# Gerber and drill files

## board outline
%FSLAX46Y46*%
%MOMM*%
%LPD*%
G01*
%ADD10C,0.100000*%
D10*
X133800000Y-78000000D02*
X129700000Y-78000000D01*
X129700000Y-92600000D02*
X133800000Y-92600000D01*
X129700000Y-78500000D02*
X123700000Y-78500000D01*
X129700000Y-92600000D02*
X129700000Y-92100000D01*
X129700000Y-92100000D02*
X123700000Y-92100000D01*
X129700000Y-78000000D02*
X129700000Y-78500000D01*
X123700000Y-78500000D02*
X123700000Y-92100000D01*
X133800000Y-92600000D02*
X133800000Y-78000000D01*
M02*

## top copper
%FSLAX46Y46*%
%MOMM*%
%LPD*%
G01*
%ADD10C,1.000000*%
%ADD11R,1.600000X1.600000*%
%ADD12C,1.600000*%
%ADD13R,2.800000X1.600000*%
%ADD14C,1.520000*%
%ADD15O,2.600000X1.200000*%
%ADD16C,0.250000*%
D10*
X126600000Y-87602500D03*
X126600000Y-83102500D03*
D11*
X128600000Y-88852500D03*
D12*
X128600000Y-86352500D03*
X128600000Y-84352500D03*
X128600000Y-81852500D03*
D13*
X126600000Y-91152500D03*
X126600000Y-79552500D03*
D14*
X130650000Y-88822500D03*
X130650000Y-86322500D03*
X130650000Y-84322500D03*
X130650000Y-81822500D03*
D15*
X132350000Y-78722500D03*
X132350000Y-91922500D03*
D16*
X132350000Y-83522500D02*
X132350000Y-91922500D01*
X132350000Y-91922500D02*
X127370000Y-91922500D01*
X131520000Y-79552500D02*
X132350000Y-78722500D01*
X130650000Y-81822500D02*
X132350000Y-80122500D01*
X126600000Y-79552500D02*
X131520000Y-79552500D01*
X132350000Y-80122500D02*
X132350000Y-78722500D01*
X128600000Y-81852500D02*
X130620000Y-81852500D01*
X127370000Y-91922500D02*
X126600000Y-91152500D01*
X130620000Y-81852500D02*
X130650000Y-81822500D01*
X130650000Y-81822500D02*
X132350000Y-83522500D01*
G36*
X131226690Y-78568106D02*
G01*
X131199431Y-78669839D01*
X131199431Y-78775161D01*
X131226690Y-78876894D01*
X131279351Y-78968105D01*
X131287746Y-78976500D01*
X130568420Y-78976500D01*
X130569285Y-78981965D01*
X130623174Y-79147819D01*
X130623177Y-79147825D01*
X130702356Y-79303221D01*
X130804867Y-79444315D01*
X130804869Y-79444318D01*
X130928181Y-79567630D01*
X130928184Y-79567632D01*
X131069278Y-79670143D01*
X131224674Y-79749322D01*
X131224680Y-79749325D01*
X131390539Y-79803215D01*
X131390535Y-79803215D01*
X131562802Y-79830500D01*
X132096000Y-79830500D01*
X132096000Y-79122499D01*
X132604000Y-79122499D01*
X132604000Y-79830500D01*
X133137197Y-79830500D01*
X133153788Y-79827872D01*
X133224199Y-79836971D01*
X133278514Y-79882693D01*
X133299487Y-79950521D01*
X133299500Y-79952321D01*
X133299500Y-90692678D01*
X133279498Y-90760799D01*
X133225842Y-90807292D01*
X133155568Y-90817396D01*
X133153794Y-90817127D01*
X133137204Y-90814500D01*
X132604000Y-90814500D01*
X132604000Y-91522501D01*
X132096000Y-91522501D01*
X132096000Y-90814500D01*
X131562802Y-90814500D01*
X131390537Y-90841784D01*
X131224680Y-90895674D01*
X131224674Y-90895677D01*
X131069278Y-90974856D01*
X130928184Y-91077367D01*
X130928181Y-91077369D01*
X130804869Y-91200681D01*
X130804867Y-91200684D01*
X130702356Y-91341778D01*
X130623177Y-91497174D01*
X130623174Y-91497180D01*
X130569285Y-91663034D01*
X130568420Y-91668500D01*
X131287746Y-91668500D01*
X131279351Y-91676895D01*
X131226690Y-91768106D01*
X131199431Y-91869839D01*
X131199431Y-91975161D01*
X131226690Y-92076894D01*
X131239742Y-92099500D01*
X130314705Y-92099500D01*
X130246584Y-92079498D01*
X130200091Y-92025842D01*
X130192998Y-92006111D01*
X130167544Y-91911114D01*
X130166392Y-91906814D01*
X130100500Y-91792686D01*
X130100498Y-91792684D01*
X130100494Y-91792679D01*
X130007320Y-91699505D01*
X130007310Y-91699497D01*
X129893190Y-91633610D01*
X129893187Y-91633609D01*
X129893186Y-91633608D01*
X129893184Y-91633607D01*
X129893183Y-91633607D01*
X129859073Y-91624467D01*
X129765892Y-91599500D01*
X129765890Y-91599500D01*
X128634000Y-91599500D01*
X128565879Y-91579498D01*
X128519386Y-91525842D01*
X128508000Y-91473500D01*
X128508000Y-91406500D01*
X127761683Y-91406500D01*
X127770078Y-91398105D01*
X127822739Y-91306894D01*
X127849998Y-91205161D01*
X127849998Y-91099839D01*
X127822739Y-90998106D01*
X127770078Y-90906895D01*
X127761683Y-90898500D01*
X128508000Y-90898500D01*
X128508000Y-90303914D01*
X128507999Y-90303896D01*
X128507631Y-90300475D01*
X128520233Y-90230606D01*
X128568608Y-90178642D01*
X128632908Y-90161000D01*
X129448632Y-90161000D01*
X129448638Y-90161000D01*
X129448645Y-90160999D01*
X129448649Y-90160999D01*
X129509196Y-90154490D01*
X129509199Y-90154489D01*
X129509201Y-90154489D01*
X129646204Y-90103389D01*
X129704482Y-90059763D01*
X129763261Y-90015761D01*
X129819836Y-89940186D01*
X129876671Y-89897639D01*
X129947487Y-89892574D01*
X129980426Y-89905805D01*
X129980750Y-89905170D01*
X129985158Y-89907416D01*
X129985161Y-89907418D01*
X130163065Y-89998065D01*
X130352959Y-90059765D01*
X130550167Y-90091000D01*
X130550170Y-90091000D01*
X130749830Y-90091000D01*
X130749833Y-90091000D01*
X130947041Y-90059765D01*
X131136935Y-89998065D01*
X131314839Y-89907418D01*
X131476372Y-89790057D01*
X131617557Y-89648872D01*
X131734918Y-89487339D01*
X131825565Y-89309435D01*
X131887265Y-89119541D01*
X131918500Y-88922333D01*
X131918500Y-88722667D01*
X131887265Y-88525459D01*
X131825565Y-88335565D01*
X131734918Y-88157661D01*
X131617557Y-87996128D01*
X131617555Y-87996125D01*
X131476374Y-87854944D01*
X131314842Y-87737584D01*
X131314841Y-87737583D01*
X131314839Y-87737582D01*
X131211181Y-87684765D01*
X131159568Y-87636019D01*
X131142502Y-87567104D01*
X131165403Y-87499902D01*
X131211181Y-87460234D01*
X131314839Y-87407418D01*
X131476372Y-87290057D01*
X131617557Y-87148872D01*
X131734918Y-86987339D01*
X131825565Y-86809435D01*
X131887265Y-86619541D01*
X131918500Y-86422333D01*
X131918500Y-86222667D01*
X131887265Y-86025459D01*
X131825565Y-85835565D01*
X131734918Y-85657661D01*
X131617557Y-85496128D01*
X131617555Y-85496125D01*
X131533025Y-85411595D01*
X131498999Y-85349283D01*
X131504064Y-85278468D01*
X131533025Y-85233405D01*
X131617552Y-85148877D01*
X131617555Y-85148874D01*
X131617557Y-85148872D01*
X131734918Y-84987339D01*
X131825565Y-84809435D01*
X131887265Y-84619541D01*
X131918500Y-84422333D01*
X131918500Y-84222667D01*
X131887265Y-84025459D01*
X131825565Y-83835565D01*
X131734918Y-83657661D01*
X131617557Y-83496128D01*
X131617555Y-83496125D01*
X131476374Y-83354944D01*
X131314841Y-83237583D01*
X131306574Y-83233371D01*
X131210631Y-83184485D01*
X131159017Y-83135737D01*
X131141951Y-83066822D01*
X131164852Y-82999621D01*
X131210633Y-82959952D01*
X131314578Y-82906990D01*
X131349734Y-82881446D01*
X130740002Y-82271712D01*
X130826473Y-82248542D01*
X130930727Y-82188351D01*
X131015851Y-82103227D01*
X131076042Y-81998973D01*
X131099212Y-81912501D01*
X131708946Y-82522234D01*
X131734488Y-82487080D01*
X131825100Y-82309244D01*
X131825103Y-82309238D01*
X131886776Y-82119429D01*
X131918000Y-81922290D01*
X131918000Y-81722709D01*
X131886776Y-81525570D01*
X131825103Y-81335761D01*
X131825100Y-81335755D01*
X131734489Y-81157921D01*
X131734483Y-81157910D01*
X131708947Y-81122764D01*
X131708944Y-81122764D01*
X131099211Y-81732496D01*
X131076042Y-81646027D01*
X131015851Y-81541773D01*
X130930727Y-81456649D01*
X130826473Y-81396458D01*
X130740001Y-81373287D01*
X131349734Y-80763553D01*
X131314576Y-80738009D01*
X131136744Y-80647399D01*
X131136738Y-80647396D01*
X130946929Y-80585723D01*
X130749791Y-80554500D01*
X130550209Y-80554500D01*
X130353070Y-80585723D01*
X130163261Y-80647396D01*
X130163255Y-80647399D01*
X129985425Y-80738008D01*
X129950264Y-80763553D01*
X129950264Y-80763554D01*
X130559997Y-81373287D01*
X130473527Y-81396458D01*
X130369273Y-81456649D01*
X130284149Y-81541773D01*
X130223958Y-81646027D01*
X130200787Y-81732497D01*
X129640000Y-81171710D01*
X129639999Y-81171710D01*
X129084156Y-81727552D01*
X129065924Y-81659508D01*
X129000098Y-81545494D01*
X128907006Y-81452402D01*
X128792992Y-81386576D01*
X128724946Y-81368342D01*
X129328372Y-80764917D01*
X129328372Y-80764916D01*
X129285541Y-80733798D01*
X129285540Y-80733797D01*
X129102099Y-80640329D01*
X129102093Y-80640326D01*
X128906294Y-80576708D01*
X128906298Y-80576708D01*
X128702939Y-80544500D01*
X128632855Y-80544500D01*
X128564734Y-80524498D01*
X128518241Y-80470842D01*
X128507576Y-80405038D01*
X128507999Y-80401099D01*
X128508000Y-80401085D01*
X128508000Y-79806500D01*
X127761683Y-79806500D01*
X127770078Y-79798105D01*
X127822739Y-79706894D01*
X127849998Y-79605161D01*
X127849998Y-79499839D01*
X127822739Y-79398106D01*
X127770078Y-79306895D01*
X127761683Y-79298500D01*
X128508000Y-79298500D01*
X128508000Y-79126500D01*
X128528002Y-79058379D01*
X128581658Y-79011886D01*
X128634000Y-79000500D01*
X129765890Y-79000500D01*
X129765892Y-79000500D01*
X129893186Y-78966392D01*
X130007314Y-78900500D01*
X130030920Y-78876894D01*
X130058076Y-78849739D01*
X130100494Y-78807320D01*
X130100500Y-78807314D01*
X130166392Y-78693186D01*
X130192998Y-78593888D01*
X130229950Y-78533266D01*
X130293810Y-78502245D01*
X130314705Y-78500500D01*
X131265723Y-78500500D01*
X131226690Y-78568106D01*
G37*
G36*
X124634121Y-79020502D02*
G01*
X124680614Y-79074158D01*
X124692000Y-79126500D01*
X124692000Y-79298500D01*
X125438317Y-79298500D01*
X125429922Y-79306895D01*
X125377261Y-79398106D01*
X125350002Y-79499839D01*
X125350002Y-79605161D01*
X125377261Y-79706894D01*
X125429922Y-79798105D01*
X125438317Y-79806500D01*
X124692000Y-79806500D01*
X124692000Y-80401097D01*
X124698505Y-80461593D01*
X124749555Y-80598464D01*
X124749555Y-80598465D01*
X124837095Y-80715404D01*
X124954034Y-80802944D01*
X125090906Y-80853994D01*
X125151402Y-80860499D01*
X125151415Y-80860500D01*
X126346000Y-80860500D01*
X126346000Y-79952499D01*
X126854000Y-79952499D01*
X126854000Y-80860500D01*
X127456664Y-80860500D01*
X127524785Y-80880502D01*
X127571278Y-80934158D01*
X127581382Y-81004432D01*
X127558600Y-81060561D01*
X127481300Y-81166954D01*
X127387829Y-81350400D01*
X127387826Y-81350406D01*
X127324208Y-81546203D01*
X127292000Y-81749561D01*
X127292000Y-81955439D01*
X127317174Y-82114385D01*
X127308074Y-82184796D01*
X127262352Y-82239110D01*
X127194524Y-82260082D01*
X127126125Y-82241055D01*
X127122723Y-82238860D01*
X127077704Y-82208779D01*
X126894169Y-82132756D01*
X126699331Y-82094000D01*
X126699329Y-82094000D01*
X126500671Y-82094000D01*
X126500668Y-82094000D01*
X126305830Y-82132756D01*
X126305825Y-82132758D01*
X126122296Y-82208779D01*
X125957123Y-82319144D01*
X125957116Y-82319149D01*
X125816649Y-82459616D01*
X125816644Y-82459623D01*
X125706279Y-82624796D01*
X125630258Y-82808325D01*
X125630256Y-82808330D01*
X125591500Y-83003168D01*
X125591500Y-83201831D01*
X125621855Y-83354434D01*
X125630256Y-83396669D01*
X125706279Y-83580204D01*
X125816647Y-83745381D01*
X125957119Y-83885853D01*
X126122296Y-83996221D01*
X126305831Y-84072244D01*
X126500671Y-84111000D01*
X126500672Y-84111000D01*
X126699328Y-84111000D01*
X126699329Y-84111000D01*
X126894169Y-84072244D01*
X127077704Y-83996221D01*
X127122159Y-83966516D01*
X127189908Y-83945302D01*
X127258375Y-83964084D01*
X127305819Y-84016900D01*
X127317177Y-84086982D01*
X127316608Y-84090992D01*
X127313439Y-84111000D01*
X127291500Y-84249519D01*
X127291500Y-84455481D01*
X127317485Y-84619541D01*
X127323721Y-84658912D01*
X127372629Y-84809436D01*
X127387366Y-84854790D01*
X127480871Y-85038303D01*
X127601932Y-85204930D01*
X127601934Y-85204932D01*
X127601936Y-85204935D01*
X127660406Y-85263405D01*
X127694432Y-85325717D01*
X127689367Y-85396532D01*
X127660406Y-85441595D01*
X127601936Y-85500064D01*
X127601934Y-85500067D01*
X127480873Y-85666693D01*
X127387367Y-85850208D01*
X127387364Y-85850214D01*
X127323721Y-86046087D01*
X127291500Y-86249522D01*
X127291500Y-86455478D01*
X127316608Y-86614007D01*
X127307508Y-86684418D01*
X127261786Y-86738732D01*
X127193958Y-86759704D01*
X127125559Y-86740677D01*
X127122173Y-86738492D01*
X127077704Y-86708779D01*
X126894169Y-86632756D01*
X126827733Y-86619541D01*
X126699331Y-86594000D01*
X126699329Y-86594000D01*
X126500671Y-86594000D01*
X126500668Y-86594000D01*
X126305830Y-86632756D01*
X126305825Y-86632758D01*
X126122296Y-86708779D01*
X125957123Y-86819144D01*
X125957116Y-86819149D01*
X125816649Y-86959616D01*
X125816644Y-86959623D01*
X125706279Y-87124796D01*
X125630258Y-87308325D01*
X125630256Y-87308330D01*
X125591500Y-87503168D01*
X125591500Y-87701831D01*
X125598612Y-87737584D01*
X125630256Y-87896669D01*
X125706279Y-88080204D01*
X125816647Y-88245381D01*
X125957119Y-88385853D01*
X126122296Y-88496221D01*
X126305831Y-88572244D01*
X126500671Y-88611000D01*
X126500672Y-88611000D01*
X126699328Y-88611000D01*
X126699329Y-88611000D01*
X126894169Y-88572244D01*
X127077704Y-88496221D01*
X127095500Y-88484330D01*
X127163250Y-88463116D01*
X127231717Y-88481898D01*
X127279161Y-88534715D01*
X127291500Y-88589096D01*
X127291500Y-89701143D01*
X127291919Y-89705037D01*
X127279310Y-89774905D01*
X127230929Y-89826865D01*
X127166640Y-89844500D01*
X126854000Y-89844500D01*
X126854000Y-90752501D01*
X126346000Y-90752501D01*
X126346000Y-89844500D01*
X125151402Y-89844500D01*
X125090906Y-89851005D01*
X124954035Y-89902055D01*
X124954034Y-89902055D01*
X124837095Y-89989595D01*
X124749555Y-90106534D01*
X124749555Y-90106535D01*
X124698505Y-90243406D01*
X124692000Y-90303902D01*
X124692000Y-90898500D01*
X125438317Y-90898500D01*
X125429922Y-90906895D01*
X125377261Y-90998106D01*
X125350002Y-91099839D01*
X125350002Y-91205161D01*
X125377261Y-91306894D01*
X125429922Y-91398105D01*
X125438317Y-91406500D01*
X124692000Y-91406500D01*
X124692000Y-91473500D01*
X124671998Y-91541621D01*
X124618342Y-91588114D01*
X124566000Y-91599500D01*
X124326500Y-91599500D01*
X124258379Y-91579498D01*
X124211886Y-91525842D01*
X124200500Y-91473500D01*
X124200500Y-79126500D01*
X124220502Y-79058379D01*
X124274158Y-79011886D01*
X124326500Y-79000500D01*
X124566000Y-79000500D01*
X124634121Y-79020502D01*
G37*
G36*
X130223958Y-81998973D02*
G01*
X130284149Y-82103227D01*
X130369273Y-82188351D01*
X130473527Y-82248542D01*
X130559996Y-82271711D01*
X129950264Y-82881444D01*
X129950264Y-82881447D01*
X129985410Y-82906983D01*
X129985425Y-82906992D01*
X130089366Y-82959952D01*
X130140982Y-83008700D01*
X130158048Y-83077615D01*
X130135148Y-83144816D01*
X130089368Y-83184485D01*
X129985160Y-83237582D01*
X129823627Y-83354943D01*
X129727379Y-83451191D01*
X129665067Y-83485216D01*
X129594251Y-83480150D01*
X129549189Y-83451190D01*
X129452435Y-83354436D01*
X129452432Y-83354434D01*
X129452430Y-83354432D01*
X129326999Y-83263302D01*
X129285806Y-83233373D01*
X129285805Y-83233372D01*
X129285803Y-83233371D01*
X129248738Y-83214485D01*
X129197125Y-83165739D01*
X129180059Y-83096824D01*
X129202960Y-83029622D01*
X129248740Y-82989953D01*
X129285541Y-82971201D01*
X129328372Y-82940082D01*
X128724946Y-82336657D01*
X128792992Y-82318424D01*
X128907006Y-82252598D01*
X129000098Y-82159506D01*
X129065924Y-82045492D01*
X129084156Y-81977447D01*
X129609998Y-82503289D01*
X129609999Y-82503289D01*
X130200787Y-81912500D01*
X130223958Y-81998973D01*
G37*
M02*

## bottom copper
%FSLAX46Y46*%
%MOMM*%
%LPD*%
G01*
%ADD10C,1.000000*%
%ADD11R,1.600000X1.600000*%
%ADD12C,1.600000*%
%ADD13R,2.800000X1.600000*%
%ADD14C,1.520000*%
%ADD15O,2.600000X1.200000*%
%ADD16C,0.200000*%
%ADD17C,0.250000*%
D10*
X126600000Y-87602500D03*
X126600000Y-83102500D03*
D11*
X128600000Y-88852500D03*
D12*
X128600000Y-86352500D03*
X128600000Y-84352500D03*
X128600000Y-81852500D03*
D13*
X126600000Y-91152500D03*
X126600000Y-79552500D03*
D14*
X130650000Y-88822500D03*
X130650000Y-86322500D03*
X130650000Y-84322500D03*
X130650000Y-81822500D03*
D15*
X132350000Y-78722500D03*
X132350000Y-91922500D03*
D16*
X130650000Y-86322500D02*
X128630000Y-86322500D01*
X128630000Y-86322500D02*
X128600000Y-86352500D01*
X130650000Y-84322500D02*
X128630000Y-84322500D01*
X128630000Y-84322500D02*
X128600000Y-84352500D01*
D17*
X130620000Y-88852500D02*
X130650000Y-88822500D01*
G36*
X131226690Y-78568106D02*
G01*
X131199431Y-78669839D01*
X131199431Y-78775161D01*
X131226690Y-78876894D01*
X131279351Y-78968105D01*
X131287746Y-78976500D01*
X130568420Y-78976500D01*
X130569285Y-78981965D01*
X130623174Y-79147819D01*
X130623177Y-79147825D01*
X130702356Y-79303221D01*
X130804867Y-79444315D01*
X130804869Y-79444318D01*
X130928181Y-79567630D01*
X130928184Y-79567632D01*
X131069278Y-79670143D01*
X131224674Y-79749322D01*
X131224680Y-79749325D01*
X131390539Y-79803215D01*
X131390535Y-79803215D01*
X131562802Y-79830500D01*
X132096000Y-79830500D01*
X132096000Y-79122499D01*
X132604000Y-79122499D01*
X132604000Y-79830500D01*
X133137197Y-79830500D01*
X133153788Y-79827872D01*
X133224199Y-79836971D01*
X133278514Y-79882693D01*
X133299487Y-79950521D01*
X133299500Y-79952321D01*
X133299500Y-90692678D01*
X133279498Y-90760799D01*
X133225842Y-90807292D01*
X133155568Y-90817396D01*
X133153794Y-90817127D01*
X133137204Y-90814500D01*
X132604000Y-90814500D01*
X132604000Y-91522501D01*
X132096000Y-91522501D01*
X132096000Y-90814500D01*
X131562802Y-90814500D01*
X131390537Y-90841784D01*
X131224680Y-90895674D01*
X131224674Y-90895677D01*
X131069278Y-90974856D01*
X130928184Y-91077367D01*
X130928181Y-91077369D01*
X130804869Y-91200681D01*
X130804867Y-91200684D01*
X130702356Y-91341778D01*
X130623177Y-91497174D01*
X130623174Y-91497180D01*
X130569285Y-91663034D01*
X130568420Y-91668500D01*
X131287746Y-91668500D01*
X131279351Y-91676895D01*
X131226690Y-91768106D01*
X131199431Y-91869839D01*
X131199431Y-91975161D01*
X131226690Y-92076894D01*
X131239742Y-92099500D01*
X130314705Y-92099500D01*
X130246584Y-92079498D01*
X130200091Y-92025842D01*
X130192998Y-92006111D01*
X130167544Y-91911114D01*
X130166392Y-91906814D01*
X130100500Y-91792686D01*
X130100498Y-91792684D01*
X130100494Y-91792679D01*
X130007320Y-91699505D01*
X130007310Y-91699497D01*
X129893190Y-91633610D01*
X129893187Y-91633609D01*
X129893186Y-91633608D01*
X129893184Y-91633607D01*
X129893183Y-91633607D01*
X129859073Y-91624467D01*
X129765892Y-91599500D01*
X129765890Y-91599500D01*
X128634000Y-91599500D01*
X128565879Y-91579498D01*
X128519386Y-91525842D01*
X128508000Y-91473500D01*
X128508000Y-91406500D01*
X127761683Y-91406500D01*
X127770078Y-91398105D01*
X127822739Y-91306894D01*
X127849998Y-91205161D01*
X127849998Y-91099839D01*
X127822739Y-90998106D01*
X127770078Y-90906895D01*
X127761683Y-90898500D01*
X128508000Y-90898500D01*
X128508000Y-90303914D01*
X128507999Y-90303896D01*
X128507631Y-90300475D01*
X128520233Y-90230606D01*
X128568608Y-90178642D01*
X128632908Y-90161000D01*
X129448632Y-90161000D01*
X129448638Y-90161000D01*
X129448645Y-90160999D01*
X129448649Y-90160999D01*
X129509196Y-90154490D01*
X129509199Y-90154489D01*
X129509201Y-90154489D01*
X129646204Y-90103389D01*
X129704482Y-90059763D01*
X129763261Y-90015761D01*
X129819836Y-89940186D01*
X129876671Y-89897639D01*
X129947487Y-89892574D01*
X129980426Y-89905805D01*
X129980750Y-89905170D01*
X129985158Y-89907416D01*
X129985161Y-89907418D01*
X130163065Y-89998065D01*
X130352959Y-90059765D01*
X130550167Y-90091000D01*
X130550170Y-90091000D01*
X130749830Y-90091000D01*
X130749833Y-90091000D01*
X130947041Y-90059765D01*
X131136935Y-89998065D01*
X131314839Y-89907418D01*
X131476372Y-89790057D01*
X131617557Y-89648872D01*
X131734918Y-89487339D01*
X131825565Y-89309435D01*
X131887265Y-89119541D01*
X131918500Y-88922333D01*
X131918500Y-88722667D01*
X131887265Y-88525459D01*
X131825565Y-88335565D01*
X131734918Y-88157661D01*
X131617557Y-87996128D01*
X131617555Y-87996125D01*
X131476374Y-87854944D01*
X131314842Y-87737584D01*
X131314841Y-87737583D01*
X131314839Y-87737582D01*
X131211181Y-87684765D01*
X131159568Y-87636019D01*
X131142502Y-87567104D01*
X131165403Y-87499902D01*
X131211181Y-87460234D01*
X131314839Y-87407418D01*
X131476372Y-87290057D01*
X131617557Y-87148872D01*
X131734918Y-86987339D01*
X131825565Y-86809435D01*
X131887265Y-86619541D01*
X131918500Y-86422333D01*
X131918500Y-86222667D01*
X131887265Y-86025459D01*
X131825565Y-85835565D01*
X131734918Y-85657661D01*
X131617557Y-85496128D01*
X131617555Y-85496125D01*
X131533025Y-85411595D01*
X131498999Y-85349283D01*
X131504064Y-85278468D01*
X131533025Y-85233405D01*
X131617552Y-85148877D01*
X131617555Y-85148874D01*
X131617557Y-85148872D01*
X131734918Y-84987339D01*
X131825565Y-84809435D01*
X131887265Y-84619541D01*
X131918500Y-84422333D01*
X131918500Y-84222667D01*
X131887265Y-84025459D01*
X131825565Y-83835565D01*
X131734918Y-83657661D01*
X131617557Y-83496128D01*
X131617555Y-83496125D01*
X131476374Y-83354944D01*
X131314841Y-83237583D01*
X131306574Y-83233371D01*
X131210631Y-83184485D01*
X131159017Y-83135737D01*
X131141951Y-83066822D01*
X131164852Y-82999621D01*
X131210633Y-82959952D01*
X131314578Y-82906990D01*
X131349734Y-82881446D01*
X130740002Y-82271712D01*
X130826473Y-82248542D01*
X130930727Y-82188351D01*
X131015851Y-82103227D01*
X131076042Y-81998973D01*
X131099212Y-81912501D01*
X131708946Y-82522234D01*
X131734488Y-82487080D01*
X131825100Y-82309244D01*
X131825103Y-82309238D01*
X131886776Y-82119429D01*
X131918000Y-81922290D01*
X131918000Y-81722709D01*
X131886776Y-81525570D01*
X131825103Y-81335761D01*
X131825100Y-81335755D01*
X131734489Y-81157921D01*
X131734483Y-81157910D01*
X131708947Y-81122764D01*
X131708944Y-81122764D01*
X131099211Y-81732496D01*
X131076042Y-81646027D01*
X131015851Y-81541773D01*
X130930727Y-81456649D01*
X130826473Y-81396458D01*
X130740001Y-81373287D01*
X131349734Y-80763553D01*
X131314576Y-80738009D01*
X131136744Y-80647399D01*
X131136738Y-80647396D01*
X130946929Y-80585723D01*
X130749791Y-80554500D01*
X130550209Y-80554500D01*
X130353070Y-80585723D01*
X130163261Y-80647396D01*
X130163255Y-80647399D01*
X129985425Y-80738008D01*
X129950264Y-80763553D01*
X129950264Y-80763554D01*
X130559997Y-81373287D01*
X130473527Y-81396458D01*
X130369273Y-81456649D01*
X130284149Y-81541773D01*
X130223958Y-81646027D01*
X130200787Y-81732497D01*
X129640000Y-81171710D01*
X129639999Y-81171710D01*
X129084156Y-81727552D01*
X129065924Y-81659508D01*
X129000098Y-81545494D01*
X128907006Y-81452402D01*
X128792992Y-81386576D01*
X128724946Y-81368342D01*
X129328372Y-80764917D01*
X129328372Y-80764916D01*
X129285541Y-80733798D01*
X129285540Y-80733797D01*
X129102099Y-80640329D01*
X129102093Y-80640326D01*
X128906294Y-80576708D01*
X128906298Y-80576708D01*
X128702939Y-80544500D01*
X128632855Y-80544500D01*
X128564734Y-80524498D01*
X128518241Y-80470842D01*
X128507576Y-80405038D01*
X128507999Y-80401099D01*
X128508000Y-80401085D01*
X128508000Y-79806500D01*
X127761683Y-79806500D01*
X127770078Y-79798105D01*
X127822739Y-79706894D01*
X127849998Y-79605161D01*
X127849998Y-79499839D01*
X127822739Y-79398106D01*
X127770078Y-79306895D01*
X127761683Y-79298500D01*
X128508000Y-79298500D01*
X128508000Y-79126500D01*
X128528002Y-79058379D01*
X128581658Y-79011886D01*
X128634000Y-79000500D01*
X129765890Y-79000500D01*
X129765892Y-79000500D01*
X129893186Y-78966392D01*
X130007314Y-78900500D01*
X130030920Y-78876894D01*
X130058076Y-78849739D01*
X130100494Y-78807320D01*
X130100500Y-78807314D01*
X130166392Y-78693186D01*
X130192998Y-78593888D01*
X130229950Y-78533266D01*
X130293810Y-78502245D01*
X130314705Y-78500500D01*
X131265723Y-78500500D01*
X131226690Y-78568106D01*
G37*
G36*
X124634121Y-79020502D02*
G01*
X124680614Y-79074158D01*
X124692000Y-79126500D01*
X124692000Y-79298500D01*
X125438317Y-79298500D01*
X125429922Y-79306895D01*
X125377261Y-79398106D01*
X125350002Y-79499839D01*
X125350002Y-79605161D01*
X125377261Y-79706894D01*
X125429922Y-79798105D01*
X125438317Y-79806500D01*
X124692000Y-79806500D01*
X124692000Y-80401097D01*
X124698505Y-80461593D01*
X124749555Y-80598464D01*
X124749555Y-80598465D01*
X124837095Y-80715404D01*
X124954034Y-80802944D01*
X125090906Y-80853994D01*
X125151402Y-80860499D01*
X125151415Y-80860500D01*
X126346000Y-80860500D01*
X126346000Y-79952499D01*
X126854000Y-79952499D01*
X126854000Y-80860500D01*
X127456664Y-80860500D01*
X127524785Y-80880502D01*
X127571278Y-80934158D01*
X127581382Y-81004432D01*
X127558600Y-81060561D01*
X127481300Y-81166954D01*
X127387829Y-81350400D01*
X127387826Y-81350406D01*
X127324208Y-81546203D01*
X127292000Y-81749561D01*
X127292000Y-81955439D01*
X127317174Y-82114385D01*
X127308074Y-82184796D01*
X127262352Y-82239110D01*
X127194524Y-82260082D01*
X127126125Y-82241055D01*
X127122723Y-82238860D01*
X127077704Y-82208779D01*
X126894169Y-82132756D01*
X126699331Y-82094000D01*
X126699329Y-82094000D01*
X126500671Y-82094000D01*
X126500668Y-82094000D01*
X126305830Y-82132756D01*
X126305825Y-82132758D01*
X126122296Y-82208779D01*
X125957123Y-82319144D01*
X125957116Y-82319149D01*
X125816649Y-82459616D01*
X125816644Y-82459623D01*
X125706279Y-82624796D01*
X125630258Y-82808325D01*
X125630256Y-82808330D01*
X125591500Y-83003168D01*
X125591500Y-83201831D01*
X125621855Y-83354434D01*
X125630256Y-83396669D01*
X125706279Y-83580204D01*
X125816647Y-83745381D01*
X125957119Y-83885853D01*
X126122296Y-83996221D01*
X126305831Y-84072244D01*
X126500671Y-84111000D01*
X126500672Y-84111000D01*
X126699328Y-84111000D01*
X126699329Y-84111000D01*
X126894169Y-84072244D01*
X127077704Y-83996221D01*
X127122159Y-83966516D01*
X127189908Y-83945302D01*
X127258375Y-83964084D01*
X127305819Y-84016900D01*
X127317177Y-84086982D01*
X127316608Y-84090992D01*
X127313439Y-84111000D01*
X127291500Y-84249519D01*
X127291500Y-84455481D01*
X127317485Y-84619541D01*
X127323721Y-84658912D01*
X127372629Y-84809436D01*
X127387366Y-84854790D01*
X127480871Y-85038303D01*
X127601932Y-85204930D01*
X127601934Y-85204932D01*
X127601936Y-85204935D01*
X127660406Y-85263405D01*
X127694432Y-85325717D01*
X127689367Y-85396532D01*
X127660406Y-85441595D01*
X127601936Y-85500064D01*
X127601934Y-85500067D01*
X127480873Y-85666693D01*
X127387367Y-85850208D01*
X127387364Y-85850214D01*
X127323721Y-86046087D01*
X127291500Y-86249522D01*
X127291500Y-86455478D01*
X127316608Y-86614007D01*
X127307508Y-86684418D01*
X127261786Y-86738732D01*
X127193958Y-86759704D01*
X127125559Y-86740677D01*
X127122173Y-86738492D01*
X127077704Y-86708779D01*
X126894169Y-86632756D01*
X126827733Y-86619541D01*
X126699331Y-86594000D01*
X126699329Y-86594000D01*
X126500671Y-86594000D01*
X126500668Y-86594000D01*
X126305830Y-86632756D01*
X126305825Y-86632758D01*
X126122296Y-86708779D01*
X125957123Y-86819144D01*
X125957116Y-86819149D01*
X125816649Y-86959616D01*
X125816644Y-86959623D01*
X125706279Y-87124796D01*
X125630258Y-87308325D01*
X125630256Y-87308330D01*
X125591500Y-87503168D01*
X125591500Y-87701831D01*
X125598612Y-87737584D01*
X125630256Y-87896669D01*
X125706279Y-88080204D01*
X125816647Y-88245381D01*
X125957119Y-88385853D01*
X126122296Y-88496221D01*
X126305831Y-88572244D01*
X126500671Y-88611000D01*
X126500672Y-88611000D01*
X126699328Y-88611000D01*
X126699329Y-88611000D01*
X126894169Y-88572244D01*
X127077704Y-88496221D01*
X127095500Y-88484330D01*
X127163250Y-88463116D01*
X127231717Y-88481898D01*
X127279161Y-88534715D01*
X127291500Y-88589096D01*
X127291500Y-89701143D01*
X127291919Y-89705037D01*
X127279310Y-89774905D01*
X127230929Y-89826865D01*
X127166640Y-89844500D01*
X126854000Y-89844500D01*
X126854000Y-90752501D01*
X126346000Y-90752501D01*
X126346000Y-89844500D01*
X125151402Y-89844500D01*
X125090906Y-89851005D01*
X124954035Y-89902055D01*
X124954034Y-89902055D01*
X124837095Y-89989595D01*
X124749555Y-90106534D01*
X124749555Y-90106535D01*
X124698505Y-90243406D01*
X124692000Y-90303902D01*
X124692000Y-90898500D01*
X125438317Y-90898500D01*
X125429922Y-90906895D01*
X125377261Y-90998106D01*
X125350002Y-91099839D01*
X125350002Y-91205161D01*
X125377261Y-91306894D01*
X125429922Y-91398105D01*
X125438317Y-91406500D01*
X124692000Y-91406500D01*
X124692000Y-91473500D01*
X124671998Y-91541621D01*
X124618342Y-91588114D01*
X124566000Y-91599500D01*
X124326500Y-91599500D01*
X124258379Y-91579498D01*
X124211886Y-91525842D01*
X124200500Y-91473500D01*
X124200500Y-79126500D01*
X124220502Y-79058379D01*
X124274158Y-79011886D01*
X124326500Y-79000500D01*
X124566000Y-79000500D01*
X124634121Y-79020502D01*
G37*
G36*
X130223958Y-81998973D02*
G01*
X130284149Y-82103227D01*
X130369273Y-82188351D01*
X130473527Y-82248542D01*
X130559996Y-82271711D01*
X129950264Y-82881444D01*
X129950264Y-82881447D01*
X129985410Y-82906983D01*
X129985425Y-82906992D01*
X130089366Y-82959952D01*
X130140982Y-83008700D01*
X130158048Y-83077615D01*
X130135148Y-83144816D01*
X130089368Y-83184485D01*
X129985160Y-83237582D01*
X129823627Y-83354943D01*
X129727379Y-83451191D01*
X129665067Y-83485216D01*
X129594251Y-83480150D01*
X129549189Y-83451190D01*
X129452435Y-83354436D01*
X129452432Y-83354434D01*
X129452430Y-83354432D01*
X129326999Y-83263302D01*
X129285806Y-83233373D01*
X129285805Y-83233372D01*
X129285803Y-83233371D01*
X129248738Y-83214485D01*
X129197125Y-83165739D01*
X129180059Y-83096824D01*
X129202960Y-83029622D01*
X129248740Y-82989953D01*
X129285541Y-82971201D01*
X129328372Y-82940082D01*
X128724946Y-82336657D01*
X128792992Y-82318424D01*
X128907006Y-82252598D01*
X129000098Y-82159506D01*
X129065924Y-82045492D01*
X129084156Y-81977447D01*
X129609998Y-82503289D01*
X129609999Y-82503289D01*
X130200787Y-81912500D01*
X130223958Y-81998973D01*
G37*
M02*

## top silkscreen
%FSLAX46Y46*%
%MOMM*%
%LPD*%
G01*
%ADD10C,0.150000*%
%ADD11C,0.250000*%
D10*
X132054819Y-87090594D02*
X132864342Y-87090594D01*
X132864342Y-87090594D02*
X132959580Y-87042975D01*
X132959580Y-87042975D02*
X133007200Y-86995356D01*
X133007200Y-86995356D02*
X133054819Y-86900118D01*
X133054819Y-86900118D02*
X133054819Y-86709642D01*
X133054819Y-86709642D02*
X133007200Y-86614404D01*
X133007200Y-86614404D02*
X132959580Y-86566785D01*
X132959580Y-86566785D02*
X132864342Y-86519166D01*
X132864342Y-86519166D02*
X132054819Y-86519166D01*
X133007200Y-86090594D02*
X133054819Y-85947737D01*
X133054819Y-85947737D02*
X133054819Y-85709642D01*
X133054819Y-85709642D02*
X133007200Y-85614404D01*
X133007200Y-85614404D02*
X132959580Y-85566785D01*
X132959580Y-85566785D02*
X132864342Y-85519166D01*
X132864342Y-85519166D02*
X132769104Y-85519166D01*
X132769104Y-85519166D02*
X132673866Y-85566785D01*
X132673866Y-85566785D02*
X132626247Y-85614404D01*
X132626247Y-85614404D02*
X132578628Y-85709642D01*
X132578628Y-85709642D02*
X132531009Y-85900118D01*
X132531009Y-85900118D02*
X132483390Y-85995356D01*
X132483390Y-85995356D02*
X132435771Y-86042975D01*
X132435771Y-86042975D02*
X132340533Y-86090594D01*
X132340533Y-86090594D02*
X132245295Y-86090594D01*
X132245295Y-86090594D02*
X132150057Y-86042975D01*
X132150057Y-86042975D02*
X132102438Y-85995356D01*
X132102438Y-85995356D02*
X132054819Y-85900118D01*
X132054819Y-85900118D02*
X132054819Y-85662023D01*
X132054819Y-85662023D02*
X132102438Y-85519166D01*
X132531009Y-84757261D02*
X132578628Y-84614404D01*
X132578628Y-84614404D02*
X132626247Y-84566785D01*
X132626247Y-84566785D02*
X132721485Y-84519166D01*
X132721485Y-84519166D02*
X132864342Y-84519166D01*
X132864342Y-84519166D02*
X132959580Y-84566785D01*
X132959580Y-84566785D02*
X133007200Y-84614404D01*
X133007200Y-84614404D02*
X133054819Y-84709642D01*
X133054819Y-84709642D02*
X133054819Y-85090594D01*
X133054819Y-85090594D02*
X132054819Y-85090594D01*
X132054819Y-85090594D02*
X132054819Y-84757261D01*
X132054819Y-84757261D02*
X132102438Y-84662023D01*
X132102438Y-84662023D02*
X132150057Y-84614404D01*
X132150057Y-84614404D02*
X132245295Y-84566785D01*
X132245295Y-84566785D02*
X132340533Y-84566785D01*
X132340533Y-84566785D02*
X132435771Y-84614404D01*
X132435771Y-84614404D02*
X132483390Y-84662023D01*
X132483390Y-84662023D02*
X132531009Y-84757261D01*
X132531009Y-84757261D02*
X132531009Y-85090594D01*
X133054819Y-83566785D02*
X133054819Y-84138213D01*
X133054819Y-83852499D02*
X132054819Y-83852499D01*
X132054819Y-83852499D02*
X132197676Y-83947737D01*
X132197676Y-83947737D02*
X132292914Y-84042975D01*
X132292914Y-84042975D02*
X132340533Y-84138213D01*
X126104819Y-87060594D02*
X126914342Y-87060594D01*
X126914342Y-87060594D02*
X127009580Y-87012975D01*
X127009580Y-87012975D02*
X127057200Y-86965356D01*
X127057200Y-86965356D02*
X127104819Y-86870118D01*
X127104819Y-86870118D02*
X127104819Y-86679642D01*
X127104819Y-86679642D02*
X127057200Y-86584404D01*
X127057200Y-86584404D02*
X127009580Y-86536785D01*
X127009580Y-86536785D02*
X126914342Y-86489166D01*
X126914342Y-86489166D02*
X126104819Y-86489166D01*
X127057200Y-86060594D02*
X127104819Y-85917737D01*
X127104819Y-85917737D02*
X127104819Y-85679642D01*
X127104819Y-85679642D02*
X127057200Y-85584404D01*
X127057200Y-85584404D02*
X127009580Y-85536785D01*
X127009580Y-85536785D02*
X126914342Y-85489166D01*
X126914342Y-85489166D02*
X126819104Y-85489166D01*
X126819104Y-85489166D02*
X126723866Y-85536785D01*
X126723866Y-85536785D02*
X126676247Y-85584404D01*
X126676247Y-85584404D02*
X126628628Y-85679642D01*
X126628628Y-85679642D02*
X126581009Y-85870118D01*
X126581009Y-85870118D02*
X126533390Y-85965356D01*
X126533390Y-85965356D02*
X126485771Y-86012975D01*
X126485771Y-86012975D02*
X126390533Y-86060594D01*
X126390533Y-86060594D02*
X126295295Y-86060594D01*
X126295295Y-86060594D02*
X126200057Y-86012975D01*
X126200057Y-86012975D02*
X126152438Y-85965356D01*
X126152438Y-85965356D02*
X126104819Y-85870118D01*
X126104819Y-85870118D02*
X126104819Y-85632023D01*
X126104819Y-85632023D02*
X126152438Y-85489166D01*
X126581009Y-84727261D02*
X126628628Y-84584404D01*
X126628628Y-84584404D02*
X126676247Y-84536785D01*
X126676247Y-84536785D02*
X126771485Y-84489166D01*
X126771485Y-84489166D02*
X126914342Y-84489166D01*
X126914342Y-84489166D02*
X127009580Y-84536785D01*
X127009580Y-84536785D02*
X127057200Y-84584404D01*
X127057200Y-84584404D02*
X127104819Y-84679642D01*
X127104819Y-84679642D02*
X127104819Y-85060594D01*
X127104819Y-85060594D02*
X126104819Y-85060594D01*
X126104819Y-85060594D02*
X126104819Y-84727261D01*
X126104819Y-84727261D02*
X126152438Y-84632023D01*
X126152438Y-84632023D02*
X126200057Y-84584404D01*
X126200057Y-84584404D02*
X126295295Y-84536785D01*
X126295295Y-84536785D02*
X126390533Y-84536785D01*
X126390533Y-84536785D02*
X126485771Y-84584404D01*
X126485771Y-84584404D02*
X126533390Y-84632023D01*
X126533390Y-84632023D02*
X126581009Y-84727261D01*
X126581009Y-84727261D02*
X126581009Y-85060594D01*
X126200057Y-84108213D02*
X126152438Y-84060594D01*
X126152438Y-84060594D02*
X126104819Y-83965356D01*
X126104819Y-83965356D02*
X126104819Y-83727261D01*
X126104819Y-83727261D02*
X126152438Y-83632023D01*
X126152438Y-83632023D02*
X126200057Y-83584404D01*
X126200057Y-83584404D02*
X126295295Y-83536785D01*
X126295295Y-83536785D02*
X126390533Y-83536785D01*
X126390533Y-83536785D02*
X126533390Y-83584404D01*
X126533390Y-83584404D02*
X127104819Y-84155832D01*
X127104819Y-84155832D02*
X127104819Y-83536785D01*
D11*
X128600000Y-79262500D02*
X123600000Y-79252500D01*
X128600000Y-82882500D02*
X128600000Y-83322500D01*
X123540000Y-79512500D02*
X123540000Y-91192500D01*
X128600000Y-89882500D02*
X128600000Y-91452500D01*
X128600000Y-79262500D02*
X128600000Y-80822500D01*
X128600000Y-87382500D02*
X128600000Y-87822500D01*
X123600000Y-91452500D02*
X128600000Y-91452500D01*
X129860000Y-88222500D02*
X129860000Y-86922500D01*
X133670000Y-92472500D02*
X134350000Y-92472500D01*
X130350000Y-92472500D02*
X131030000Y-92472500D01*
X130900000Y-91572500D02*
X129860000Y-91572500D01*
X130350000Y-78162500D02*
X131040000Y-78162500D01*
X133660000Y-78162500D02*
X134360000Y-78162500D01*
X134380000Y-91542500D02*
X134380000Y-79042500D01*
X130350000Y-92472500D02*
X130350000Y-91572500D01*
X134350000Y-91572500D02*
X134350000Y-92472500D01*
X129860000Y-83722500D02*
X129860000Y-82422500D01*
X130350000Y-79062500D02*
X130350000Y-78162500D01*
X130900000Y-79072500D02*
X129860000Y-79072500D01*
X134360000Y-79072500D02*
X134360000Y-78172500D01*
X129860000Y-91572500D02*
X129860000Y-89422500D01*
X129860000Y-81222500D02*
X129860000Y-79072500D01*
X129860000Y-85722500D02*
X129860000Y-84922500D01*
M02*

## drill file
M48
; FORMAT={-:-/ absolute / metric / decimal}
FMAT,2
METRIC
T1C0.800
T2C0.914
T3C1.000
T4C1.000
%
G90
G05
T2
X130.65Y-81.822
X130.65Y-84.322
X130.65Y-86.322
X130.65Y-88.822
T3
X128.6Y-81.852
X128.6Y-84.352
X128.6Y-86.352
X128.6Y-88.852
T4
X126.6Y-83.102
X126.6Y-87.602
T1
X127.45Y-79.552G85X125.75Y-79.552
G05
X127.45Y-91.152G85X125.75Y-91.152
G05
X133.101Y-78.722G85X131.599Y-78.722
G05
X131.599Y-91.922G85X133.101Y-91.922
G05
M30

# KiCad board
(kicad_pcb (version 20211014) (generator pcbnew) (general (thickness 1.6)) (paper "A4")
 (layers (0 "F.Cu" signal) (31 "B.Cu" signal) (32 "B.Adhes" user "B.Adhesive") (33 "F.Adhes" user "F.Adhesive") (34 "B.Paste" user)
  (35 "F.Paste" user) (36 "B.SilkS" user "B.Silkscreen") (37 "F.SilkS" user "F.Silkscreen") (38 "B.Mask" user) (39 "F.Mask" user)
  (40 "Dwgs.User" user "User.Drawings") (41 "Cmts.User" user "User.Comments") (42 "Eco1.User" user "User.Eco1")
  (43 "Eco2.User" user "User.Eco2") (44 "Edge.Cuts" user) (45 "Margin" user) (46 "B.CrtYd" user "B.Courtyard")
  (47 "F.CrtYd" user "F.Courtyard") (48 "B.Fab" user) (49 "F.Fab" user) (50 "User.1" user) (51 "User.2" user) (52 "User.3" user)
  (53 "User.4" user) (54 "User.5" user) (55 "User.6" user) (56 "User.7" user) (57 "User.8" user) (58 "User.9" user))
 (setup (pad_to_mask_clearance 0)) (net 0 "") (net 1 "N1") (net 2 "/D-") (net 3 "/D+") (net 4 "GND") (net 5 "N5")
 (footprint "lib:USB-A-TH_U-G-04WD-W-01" (layer "F.Cu") (at 127.6 85.3525 -90)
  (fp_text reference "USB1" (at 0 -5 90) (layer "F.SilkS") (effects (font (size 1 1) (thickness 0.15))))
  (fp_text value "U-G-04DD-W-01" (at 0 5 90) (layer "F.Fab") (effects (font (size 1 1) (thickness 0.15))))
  (fp_line (start -6.09 -1) (end -6.1 4) (layer "F.SilkS") (width 0.25))
  (fp_line (start -2.47 -1) (end -2.03 -1) (layer "F.SilkS") (width 0.25))
  (fp_line (start -5.84 4.06) (end 5.84 4.06) (layer "F.SilkS") (width 0.25))
  (fp_line (start 4.53 -1) (end 6.1 -1) (layer "F.SilkS") (width 0.25))
  (fp_line (start -6.09 -1) (end -4.53 -1) (layer "F.SilkS") (width 0.25))
  (fp_line (start 2.03 -1) (end 2.47 -1) (layer "F.SilkS") (width 0.25))
  (fp_line (start 6.1 4) (end 6.1 -1) (layer "F.SilkS") (width 0.25))
  (pad "" thru_hole circle (at 2.25 1 270) (size 1 1) (drill 1) (layers *.Cu *.Mask))
  (pad "" thru_hole circle (at -2.25 1 270) (size 1 1) (drill 1) (layers *.Cu *.Mask))
  (pad "1" thru_hole rect (at 3.5 -1 270) (size 1.6 1.6) (drill 0.999998) (layers *.Cu *.Paste *.Mask) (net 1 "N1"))
  (pad "2" thru_hole circle (at 1 -1 270) (size 1.6 1.6) (drill 0.999998) (layers *.Cu *.Paste *.Mask) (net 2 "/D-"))
  (pad "3" thru_hole circle (at -1 -1 270) (size 1.6 1.6) (drill 0.999998) (layers *.Cu *.Paste *.Mask) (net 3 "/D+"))
  (pad "4" thru_hole circle (at -3.5 -1 270) (size 1.6 1.6) (drill 0.999998) (layers *.Cu *.Paste *.Mask) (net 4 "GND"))
  (pad "5" thru_hole rect (at 5.8 1 270) (size 1.6 2.8) (drill oval 0.799998 2.499995) (layers *.Cu *.Paste *.Mask) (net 4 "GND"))
  (pad "6" thru_hole rect (at -5.8 1 270) (size 1.6 2.8) (drill oval 0.799998 2.499995) (layers *.Cu *.Paste *.Mask) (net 4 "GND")))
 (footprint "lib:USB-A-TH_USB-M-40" (layer "F.Cu") (at 131.5 85.3225 90)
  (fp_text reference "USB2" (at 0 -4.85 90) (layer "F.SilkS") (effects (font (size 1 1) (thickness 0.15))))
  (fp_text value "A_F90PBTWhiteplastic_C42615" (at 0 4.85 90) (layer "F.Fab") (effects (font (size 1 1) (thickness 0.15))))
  (fp_line (start -2.9 -1.64) (end -1.6 -1.64) (layer "F.SilkS") (width 0.25))
  (fp_line (start -7.15 2.17) (end -7.15 2.85) (layer "F.SilkS") (width 0.25))
  (fp_line (start -7.15 -1.15) (end -7.15 -0.47) (layer "F.SilkS") (width 0.25))
  (fp_line (start -6.25 -0.6) (end -6.25 -1.64) (layer "F.SilkS") (width 0.25))
  (fp_line (start 7.16 -1.15) (end 7.16 -0.46) (layer "F.SilkS") (width 0.25))
  (fp_line (start 7.16 2.16) (end 7.16 2.86) (layer "F.SilkS") (width 0.25))
  (fp_line (start -6.22 2.88) (end 6.28 2.88) (layer "F.SilkS") (width 0.25))
  (fp_line (start -7.15 -1.15) (end -6.25 -1.15) (layer "F.SilkS") (width 0.25))
  (fp_line (start -6.25 2.85) (end -7.15 2.85) (layer "F.SilkS") (width 0.25))
  (fp_line (start 1.6 -1.64) (end 2.9 -1.64) (layer "F.SilkS") (width 0.25))
  (fp_line (start 6.26 -1.15) (end 7.16 -1.15) (layer "F.SilkS") (width 0.25))
  (fp_line (start 6.25 -0.6) (end 6.25 -1.64) (layer "F.SilkS") (width 0.25))
  (fp_line (start 6.25 2.86) (end 7.15 2.86) (layer "F.SilkS") (width 0.25))
  (fp_line (start -6.25 -1.64) (end -4.1 -1.64) (layer "F.SilkS") (width 0.25))
  (fp_line (start 4.1 -1.64) (end 6.25 -1.64) (layer "F.SilkS") (width 0.25))
  (fp_line (start -0.4 -1.64) (end 0.4 -1.64) (layer "F.SilkS") (width 0.25))
  (pad "1" thru_hole circle (at -3.5 -0.85 90) (size 1.52 1.52) (drill 0.9144) (layers *.Cu *.Paste *.Mask) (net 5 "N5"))
  (pad "2" thru_hole circle (at -1 -0.85 90) (size 1.52 1.52) (drill 0.9144) (layers *.Cu *.Paste *.Mask) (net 2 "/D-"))
  (pad "3" thru_hole circle (at 1 -0.85 90) (size 1.52 1.52) (drill 0.9144) (layers *.Cu *.Paste *.Mask) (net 3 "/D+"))
  (pad "4" thru_hole circle (at 3.5 -0.85 90) (size 1.52 1.52) (drill 0.9144) (layers *.Cu *.Paste *.Mask) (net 4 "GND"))
  (pad "5" thru_hole oval (at 6.6 0.85 180) (size 2.6 1.2) (drill oval 2.301138 0.799998) (layers *.Cu *.Paste *.Mask) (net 4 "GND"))
  (pad "6" thru_hole oval (at -6.6 0.85) (size 2.6 1.2) (drill oval 2.301138 0.799998) (layers *.Cu *.Paste *.Mask) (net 4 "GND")))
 (gr_line (start 133.8 78) (end 129.7 78) (layer "Edge.Cuts") (width 0.1))
 (gr_line (start 129.7 92.6) (end 133.8 92.6) (layer "Edge.Cuts") (width 0.1))
 (gr_line (start 129.7 78.5) (end 123.7 78.5) (layer "Edge.Cuts") (width 0.1))
 (gr_line (start 129.7 92.6) (end 129.7 92.1) (layer "Edge.Cuts") (width 0.1))
 (gr_line (start 129.7 92.1) (end 123.7 92.1) (layer "Edge.Cuts") (width 0.1))
 (gr_line (start 129.7 78) (end 129.7 78.5) (layer "Edge.Cuts") (width 0.1))
 (gr_line (start 123.7 78.5) (end 123.7 92.1) (layer "Edge.Cuts") (width 0.1))
 (gr_line (start 133.8 92.6) (end 133.8 78) (layer "Edge.Cuts") (width 0.1))
 (segment (start 132.35 83.5225) (end 132.35 91.9225) (width 0.25) (layer "F.Cu") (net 4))
 (segment (start 132.35 91.9225) (end 127.37 91.9225) (width 0.25) (layer "F.Cu") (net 4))
 (segment (start 131.52 79.5525) (end 132.35 78.7225) (width 0.25) (layer "F.Cu") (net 4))
 (segment (start 130.65 81.8225) (end 132.35 80.1225) (width 0.25) (layer "F.Cu") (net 4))
 (segment (start 126.6 79.5525) (end 131.52 79.5525) (width 0.25) (layer "F.Cu") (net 4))
 (segment (start 132.35 80.1225) (end 132.35 78.7225) (width 0.25) (layer "F.Cu") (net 4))
 (segment (start 128.6 81.8525) (end 130.62 81.8525) (width 0.25) (layer "F.Cu") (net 4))
 (segment (start 127.37 91.9225) (end 126.6 91.1525) (width 0.25) (layer "F.Cu") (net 4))
 (segment (start 130.62 81.8525) (end 130.65 81.8225) (width 0.25) (layer "F.Cu") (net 4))
 (segment (start 130.65 81.8225) (end 132.35 83.5225) (width 0.25) (layer "F.Cu") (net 4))
 (segment (start 130.65 86.3225) (end 128.63 86.3225) (width 0.2) (layer "B.Cu") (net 2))
 (segment (start 128.63 86.3225) (end 128.6 86.3525) (width 0.2) (layer "B.Cu") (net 2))
 (segment (start 130.65 84.3225) (end 128.63 84.3225) (width 0.2) (layer "B.Cu") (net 3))
 (segment (start 128.63 84.3225) (end 128.6 84.3525) (width 0.2) (layer "B.Cu") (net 3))
 (segment (start 130.62 88.8525) (end 130.65 88.8225) (width 0.25) (layer "B.Cu") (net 5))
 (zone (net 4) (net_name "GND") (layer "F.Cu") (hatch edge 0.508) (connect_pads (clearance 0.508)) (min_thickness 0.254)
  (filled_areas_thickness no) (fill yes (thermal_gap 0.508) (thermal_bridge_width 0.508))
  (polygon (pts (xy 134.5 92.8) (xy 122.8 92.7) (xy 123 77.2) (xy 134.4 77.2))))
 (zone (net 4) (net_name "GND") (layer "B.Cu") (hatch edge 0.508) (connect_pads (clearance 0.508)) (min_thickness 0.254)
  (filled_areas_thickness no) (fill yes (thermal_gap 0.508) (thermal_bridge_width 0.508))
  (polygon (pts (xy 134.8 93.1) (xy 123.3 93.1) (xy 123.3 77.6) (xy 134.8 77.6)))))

